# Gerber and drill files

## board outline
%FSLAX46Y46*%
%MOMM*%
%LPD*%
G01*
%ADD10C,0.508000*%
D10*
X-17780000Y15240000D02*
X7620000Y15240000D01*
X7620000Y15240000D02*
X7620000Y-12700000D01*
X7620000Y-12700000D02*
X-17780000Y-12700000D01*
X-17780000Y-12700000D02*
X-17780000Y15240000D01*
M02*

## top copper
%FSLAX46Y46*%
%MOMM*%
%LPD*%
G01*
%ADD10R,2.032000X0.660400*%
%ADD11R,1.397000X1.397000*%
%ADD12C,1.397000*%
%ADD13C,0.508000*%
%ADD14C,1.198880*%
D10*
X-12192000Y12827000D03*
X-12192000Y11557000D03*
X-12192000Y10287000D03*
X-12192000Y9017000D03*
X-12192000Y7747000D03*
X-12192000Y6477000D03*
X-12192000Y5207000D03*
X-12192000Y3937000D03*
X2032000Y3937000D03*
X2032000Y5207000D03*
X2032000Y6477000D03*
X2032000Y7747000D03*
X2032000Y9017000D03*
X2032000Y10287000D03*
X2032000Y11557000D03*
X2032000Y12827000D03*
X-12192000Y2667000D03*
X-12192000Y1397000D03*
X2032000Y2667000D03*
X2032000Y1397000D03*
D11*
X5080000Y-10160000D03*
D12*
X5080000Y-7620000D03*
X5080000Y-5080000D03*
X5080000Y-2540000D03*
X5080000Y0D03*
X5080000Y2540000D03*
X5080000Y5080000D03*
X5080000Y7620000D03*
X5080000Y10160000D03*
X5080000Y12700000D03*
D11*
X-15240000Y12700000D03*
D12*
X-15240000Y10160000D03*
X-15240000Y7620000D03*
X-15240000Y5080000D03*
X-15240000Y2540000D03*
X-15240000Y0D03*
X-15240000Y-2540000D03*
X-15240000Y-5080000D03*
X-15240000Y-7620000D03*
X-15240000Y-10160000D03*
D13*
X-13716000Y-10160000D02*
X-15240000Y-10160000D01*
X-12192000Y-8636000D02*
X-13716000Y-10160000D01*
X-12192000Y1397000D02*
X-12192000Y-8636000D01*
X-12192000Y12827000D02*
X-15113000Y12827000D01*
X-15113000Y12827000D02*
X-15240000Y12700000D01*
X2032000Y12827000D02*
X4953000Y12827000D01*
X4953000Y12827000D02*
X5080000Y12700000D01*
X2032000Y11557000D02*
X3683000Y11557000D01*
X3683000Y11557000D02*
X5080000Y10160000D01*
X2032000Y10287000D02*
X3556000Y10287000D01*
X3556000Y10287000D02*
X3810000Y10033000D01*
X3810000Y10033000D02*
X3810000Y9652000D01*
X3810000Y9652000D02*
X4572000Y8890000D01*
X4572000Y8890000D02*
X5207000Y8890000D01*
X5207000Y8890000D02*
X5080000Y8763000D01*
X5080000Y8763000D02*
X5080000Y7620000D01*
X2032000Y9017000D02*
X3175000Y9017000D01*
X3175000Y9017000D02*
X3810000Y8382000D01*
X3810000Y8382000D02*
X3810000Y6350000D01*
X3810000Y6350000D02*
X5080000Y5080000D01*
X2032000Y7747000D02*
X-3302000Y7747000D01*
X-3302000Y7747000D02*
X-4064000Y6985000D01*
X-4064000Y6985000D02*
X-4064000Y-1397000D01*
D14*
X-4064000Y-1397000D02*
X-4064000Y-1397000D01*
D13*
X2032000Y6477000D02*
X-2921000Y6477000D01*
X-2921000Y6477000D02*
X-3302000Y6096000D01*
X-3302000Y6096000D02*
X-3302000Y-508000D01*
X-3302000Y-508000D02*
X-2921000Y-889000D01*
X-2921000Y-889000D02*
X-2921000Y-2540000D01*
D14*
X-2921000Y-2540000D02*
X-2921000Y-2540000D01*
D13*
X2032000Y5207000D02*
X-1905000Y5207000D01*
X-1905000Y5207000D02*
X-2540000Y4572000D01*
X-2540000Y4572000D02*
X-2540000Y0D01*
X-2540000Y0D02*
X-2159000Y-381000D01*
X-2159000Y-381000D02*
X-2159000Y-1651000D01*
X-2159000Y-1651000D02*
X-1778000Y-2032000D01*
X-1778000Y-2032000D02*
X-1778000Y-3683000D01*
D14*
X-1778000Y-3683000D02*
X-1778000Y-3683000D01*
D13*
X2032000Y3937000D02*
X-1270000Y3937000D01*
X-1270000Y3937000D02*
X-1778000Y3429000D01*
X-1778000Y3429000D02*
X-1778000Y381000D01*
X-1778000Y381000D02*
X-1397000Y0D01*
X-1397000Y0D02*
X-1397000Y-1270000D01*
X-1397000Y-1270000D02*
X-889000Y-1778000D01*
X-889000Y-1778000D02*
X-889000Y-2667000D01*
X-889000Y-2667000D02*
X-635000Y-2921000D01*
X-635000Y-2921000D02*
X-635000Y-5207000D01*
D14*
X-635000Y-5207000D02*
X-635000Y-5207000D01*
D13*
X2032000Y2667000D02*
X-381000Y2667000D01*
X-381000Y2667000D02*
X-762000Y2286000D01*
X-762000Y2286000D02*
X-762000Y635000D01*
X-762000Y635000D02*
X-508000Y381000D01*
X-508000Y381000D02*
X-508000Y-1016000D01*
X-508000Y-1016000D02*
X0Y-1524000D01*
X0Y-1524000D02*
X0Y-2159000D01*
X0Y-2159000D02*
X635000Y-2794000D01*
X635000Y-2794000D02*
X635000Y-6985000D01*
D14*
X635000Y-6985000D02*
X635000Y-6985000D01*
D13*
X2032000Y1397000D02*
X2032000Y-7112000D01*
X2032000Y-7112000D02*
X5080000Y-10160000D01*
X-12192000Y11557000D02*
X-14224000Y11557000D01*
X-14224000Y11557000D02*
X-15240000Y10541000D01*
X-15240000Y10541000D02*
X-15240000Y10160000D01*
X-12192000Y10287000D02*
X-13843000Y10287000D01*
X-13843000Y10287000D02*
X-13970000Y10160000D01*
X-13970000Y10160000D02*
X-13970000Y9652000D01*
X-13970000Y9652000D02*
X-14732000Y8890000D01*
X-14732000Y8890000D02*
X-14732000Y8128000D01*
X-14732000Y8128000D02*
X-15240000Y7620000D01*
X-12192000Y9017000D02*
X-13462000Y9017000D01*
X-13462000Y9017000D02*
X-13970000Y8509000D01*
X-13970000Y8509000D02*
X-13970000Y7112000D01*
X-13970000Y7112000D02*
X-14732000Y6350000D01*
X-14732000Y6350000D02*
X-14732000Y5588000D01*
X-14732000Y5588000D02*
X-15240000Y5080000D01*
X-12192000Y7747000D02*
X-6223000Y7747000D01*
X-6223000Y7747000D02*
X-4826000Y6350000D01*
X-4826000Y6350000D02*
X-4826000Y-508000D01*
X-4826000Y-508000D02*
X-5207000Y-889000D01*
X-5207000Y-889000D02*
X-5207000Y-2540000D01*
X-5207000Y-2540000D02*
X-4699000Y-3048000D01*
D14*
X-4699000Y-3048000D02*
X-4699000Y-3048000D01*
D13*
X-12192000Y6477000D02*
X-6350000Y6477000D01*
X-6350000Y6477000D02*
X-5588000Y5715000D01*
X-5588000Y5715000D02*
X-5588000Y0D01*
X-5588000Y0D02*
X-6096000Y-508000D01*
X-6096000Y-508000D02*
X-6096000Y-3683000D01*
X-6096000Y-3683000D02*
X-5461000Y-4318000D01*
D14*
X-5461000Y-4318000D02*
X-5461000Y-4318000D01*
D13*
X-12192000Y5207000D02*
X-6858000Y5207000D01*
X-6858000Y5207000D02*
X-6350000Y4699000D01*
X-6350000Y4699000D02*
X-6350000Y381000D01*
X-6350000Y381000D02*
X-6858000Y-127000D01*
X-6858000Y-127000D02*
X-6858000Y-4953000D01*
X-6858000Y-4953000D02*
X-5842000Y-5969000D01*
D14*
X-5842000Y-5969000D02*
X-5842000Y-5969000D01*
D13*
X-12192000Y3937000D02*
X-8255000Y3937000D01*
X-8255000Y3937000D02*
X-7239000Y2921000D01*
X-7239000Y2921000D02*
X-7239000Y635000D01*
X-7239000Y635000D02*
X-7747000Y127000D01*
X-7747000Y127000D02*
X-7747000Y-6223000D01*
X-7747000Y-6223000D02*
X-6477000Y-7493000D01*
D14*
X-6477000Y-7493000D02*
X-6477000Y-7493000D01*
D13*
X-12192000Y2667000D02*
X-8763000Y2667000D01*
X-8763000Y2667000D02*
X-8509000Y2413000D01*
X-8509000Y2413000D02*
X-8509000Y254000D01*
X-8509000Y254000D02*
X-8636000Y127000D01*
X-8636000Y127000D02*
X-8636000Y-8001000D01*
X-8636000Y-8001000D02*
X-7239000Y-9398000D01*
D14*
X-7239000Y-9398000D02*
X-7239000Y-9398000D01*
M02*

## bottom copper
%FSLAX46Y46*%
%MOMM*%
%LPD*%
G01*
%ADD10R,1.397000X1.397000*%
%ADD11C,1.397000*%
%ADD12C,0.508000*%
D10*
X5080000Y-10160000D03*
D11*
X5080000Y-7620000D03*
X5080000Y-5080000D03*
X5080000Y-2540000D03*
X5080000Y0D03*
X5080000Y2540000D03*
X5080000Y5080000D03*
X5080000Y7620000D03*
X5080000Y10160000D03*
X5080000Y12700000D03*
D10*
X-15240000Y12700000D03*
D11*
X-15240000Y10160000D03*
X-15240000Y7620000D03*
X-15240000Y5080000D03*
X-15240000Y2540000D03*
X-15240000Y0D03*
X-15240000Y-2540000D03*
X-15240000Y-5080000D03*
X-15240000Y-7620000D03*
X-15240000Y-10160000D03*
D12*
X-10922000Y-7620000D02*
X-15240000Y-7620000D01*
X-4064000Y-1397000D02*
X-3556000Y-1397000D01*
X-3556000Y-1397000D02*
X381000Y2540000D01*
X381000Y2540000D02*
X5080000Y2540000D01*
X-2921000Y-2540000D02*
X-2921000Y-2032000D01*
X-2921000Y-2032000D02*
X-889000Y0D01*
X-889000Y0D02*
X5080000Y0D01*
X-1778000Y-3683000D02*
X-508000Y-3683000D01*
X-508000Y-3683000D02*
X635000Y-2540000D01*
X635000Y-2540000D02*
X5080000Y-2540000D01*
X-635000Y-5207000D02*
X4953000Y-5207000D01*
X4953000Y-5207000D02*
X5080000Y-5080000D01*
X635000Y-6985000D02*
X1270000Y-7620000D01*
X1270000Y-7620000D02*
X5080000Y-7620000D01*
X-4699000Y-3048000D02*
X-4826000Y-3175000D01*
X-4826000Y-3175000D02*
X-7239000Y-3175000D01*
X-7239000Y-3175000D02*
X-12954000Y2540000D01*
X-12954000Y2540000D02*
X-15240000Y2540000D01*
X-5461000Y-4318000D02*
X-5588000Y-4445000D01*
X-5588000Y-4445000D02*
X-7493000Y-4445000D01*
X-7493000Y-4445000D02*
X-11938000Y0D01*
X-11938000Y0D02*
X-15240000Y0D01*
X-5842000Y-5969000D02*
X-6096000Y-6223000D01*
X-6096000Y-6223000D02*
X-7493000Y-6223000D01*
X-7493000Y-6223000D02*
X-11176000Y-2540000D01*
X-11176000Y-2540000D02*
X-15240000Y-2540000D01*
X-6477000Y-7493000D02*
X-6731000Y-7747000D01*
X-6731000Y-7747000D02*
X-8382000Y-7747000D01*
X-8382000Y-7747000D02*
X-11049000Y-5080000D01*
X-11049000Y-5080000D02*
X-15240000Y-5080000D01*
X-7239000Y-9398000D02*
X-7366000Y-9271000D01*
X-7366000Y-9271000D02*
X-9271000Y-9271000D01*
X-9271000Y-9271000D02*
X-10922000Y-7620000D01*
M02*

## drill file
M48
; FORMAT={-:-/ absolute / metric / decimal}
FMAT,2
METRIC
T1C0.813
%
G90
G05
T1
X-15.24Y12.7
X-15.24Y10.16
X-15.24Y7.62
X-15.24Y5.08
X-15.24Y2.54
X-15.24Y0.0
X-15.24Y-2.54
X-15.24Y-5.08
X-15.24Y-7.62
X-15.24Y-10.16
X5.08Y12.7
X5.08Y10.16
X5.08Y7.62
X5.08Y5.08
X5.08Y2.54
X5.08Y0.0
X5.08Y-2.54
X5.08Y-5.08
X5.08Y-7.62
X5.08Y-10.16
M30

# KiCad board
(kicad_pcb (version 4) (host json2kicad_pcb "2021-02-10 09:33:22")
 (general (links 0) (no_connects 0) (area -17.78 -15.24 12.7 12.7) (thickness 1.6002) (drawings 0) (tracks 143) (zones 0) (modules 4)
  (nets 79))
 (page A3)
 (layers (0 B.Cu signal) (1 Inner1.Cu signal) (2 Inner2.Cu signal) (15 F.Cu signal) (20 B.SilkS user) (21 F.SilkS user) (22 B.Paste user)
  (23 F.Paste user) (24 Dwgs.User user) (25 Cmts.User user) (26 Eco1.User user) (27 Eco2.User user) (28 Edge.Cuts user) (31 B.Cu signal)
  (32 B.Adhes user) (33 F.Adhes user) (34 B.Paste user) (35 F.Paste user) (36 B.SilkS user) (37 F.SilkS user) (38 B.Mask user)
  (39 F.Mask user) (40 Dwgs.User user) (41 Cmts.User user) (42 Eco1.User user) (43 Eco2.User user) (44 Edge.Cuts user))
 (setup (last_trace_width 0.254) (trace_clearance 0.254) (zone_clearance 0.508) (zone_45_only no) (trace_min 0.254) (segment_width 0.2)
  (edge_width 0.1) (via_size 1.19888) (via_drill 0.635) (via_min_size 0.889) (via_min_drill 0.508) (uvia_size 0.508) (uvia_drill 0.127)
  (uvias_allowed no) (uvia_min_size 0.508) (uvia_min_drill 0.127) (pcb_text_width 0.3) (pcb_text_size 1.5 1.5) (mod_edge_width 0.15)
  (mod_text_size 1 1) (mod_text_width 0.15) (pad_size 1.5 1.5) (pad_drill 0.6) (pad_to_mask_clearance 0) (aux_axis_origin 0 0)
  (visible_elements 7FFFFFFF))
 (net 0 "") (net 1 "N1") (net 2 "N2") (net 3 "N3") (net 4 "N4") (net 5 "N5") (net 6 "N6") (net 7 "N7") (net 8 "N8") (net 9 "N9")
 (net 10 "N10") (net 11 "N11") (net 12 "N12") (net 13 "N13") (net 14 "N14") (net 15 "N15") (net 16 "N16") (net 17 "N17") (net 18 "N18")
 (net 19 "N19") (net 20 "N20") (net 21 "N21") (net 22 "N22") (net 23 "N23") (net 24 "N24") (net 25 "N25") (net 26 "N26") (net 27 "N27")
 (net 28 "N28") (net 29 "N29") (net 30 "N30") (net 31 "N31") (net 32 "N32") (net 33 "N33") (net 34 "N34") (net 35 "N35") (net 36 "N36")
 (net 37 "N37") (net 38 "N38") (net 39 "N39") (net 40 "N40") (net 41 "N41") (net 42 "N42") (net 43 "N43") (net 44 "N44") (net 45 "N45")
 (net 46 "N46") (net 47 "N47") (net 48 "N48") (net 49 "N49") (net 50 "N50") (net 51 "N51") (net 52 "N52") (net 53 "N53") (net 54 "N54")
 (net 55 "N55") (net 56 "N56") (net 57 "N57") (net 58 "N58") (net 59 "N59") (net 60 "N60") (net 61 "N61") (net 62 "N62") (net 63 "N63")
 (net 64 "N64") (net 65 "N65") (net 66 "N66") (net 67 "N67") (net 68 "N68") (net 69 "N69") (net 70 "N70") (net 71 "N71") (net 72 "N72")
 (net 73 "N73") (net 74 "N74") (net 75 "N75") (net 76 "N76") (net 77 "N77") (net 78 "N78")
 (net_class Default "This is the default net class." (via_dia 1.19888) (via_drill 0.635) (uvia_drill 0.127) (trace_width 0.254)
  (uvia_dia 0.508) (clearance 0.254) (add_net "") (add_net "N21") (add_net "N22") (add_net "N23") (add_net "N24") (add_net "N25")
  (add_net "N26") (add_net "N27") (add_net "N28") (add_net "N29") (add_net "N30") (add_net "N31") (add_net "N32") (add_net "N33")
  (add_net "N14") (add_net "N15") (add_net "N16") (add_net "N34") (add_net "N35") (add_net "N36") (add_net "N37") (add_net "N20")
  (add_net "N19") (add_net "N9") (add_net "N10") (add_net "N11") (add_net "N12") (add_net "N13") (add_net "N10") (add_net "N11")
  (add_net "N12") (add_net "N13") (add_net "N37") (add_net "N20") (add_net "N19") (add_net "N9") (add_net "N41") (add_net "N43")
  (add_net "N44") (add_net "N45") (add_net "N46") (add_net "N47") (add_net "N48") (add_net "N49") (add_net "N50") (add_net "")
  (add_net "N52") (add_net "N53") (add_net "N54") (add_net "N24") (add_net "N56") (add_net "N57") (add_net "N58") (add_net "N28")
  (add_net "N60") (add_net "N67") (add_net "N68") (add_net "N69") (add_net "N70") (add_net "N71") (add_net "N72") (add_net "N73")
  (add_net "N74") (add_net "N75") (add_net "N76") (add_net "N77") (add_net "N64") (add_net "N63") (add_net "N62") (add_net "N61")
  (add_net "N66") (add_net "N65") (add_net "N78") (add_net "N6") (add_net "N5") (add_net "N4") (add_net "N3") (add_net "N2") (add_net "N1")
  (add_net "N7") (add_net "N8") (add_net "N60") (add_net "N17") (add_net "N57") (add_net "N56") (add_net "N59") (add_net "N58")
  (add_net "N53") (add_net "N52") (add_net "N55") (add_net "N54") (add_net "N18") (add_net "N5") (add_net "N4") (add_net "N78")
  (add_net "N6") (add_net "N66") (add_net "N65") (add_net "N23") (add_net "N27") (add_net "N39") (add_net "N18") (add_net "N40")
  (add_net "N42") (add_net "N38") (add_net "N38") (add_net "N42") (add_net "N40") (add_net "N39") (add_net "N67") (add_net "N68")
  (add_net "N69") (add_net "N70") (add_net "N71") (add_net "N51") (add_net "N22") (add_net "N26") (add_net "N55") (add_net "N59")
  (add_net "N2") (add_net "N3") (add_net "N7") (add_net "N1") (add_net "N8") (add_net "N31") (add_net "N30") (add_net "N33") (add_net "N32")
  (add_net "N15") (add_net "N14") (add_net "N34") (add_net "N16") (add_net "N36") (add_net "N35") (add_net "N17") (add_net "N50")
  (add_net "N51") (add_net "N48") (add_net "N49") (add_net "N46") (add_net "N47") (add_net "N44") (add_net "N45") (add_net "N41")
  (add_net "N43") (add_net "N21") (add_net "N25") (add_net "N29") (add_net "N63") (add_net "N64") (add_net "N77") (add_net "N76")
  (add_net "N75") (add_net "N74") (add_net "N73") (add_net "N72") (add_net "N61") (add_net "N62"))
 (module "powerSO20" (layer "F.Cu") (at -5.08 -7.112 -90.00)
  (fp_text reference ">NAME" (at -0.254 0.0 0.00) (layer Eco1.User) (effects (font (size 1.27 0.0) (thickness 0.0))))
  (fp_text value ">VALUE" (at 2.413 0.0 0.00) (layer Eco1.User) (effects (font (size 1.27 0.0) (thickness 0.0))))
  (pad 1 smd rect (at -5.715 7.112 -90.00) (size 0.6604 2.032) (drill 0.0) (layers "F.Cu" "F.Paste") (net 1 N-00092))
  (pad 2 smd rect (at -4.445 7.112 -90.00) (size 0.6604 2.032) (drill 0.0) (layers "F.Cu" "F.Paste") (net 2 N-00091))
  (pad 3 smd rect (at -3.175 7.112 -90.00) (size 0.6604 2.032) (drill 0.0) (layers "F.Cu" "F.Paste") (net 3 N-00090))
  (pad 4 smd rect (at -1.905 7.112 -90.00) (size 0.6604 2.032) (drill 0.0) (layers "F.Cu" "F.Paste") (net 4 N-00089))
  (pad 5 smd rect (at -0.635 7.112 -90.00) (size 0.6604 2.032) (drill 0.0) (layers "F.Cu" "F.Paste") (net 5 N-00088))
  (pad 6 smd rect (at 0.635 7.112 -90.00) (size 0.6604 2.032) (drill 0.0) (layers "F.Cu" "F.Paste") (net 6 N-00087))
  (pad 7 smd rect (at 1.905 7.112 -90.00) (size 0.6604 2.032) (drill 0.0) (layers "F.Cu" "F.Paste") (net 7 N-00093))
  (pad 8 smd rect (at 3.175 7.112 -90.00) (size 0.6604 2.032) (drill 0.0) (layers "F.Cu" "F.Paste") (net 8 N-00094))
  (pad 13 smd rect (at 3.175 -7.112 -90.00) (size 0.6604 2.032) (drill 0.0) (layers "F.Cu" "F.Paste") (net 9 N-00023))
  (pad 14 smd rect (at 1.905 -7.112 -90.00) (size 0.6604 2.032) (drill 0.0) (layers "F.Cu" "F.Paste") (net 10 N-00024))
  (pad 15 smd rect (at 0.635 -7.112 -90.00) (size 0.6604 2.032) (drill 0.0) (layers "F.Cu" "F.Paste") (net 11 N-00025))
  (pad 16 smd rect (at -0.635 -7.112 -90.00) (size 0.6604 2.032) (drill 0.0) (layers "F.Cu" "F.Paste") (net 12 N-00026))
  (pad 17 smd rect (at -1.905 -7.112 -90.00) (size 0.6604 2.032) (drill 0.0) (layers "F.Cu" "F.Paste") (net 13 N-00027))
  (pad 18 smd rect (at -3.175 -7.112 -90.00) (size 0.6604 2.032) (drill 0.0) (layers "F.Cu" "F.Paste") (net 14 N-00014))
  (pad 19 smd rect (at -4.445 -7.112 -90.00) (size 0.6604 2.032) (drill 0.0) (layers "F.Cu" "F.Paste") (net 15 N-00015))
  (pad 20 smd rect (at -5.715 -7.112 -90.00) (size 0.6604 2.032) (drill 0.0) (layers "F.Cu" "F.Paste") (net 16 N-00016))
  (pad 9 smd rect (at 4.445 7.112 -90.00) (size 0.6604 2.032) (drill 0.0) (layers "F.Cu" "F.Paste") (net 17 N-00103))
  (pad 10 smd rect (at 5.715 7.112 -90.00) (size 0.6604 2.032) (drill 0.0) (layers "F.Cu" "F.Paste") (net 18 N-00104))
  (pad 12 smd rect (at 4.445 -7.112 -90.00) (size 0.6604 2.032) (drill 0.0) (layers "F.Cu" "F.Paste") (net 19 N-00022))
  (pad 11 smd rect (at 5.715 -7.112 -90.00) (size 0.6604 2.032) (drill 0.0) (layers "F.Cu" "F.Paste") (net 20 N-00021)))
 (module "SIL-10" (layer "F.Cu") (at 5.08 -1.27 90.00)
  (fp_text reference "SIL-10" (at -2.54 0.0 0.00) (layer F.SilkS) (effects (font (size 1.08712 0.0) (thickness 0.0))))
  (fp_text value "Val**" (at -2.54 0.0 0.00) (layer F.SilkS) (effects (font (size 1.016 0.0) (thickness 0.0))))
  (pad 1 thru_hole rect (at -11.43 0.0 90.00) (size 1.397 1.397) (drill 0.8128)
   (layers "B.Cu" "Inner1.Cu" "Inner2.Cu" "F.Cu" "F.SilkS" "B.Paste" "F.Paste") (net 20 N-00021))
  (pad 2 thru_hole circle (at -8.89 0.0 90.00) (size 1.397 1.397) (drill 0.8128)
   (layers "B.Cu" "Inner1.Cu" "Inner2.Cu" "F.Cu" "F.SilkS" "B.Paste" "F.Paste") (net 19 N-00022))
  (pad 3 thru_hole circle (at -6.35 0.0 90.00) (size 1.397 1.397) (drill 0.8128)
   (layers "B.Cu" "Inner1.Cu" "Inner2.Cu" "F.Cu" "F.SilkS" "B.Paste" "F.Paste") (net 9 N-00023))
  (pad 4 thru_hole circle (at -3.81 0.0 90.00) (size 1.397 1.397) (drill 0.8128)
   (layers "B.Cu" "Inner1.Cu" "Inner2.Cu" "F.Cu" "F.SilkS" "B.Paste" "F.Paste") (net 10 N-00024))
  (pad 5 thru_hole circle (at -1.27 0.0 90.00) (size 1.397 1.397) (drill 0.8128)
   (layers "B.Cu" "Inner1.Cu" "Inner2.Cu" "F.Cu" "F.SilkS" "B.Paste" "F.Paste") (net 11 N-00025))
  (pad 6 thru_hole circle (at 1.27 0.0 90.00) (size 1.397 1.397) (drill 0.8128)
   (layers "B.Cu" "Inner1.Cu" "Inner2.Cu" "F.Cu" "F.SilkS" "B.Paste" "F.Paste") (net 12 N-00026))
  (pad 7 thru_hole circle (at 3.81 0.0 90.00) (size 1.397 1.397) (drill 0.8128)
   (layers "B.Cu" "Inner1.Cu" "Inner2.Cu" "F.Cu" "F.SilkS" "B.Paste" "F.Paste") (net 13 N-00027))
  (pad 8 thru_hole circle (at 6.35 0.0 90.00) (size 1.397 1.397) (drill 0.8128)
   (layers "B.Cu" "Inner1.Cu" "Inner2.Cu" "F.Cu" "F.SilkS" "B.Paste" "F.Paste") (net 14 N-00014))
  (pad 9 thru_hole circle (at 8.89 0.0 90.00) (size 1.397 1.397) (drill 0.8128)
   (layers "B.Cu" "Inner1.Cu" "Inner2.Cu" "F.Cu" "F.SilkS" "B.Paste" "F.Paste") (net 15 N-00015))
  (pad 10 thru_hole circle (at 11.43 0.0 90.00) (size 1.397 1.397) (drill 0.8128)
   (layers "B.Cu" "Inner1.Cu" "Inner2.Cu" "F.Cu" "F.SilkS" "B.Paste" "F.Paste") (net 16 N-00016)))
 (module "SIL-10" (layer "F.Cu") (at -15.24 -1.27 -90.00)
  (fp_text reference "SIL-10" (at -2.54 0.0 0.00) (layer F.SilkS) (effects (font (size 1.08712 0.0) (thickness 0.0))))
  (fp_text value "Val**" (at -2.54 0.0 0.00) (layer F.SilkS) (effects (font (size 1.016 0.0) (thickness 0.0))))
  (pad 1 thru_hole rect (at -11.43 0.0 -90.00) (size 1.397 1.397) (drill 0.8128)
   (layers "B.Cu" "Inner1.Cu" "Inner2.Cu" "F.Cu" "F.SilkS" "B.Paste" "F.Paste") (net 1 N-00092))
  (pad 2 thru_hole circle (at -8.89 0.0 -90.00) (size 1.397 1.397) (drill 0.8128)
   (layers "B.Cu" "Inner1.Cu" "Inner2.Cu" "F.Cu" "F.SilkS" "B.Paste" "F.Paste") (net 2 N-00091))
  (pad 3 thru_hole circle (at -6.35 0.0 -90.00) (size 1.397 1.397) (drill 0.8128)
   (layers "B.Cu" "Inner1.Cu" "Inner2.Cu" "F.Cu" "F.SilkS" "B.Paste" "F.Paste") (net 3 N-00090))
  (pad 4 thru_hole circle (at -3.81 0.0 -90.00) (size 1.397 1.397) (drill 0.8128)
   (layers "B.Cu" "Inner1.Cu" "Inner2.Cu" "F.Cu" "F.SilkS" "B.Paste" "F.Paste") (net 4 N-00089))
  (pad 5 thru_hole circle (at -1.27 0.0 -90.00) (size 1.397 1.397) (drill 0.8128)
   (layers "B.Cu" "Inner1.Cu" "Inner2.Cu" "F.Cu" "F.SilkS" "B.Paste" "F.Paste") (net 5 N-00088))
  (pad 6 thru_hole circle (at 1.27 0.0 -90.00) (size 1.397 1.397) (drill 0.8128)
   (layers "B.Cu" "Inner1.Cu" "Inner2.Cu" "F.Cu" "F.SilkS" "B.Paste" "F.Paste") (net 6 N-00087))
  (pad 7 thru_hole circle (at 3.81 0.0 -90.00) (size 1.397 1.397) (drill 0.8128)
   (layers "B.Cu" "Inner1.Cu" "Inner2.Cu" "F.Cu" "F.SilkS" "B.Paste" "F.Paste") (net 7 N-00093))
  (pad 8 thru_hole circle (at 6.35 0.0 -90.00) (size 1.397 1.397) (drill 0.8128)
   (layers "B.Cu" "Inner1.Cu" "Inner2.Cu" "F.Cu" "F.SilkS" "B.Paste" "F.Paste") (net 8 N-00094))
  (pad 9 thru_hole circle (at 8.89 0.0 -90.00) (size 1.397 1.397) (drill 0.8128)
   (layers "B.Cu" "Inner1.Cu" "Inner2.Cu" "F.Cu" "F.SilkS" "B.Paste" "F.Paste") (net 17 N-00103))
  (pad 10 thru_hole circle (at 11.43 0.0 -90.00) (size 1.397 1.397) (drill 0.8128)
   (layers "B.Cu" "Inner1.Cu" "Inner2.Cu" "F.Cu" "F.SilkS" "B.Paste" "F.Paste") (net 18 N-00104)))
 (segment (start -13.716 10.16) (end -15.24 10.16) (width 0.508) (layer F.Cu) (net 18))
 (segment (start -12.192 8.636) (end -13.716 10.16) (width 0.508) (layer F.Cu) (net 18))
 (segment (start -12.192 -1.397) (end -12.192 8.636) (width 0.508) (layer F.Cu) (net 18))
 (segment (start -10.922 7.62) (end -15.24 7.62) (width 0.508) (layer B.Cu) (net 17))
 (segment (start -12.192 -12.827) (end -15.113 -12.827) (width 0.508) (layer F.Cu) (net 1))
 (segment (start -15.113 -12.827) (end -15.24 -12.7) (width 0.508) (layer F.Cu) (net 1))
 (segment (start 2.032 -12.827) (end 4.953 -12.827) (width 0.508) (layer F.Cu) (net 16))
 (segment (start 4.953 -12.827) (end 5.08 -12.7) (width 0.508) (layer F.Cu) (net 16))
 (segment (start 2.032 -11.557) (end 3.683 -11.557) (width 0.508) (layer F.Cu) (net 15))
 (segment (start 3.683 -11.557) (end 5.08 -10.16) (width 0.508) (layer F.Cu) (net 15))
 (segment (start 2.032 -10.287) (end 3.556 -10.287) (width 0.508) (layer F.Cu) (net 14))
 (segment (start 3.556 -10.287) (end 3.81 -10.033) (width 0.508) (layer F.Cu) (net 14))
 (segment (start 3.81 -10.033) (end 3.81 -9.652) (width 0.508) (layer F.Cu) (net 14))
 (segment (start 3.81 -9.652) (end 4.572 -8.89) (width 0.508) (layer F.Cu) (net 14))
 (segment (start 4.572 -8.89) (end 5.207 -8.89) (width 0.508) (layer F.Cu) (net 14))
 (segment (start 5.207 -8.89) (end 5.08 -8.763) (width 0.508) (layer F.Cu) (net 14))
 (segment (start 5.08 -8.763) (end 5.08 -7.62) (width 0.508) (layer F.Cu) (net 14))
 (segment (start 2.032 -9.017) (end 3.175 -9.017) (width 0.508) (layer F.Cu) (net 13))
 (segment (start 3.175 -9.017) (end 3.81 -8.382) (width 0.508) (layer F.Cu) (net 13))
 (segment (start 3.81 -8.382) (end 3.81 -6.35) (width 0.508) (layer F.Cu) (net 13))
 (segment (start 3.81 -6.35) (end 5.08 -5.08) (width 0.508) (layer F.Cu) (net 13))
 (segment (start 2.032 -7.747) (end -3.302 -7.747) (width 0.508) (layer F.Cu) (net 12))
 (segment (start -3.302 -7.747) (end -4.064 -6.985) (width 0.508) (layer F.Cu) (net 12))
 (segment (start -4.064 -6.985) (end -4.064 1.397) (width 0.508) (layer F.Cu) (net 12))
 (segment (start -4.064 1.397) (end -4.064 1.397) (width 1.19888) (layer F.Cu) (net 12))
 (segment (start -4.064 1.397) (end -3.556 1.397) (width 0.508) (layer B.Cu) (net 12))
 (segment (start -3.556 1.397) (end 0.381 -2.54) (width 0.508) (layer B.Cu) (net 12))
 (segment (start 0.381 -2.54) (end 5.08 -2.54) (width 0.508) (layer B.Cu) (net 12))
 (segment (start 2.032 -6.477) (end -2.921 -6.477) (width 0.508) (layer F.Cu) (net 11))
 (segment (start -2.921 -6.477) (end -3.302 -6.096) (width 0.508) (layer F.Cu) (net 11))
 (segment (start -3.302 -6.096) (end -3.302 0.508) (width 0.508) (layer F.Cu) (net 11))
 (segment (start -3.302 0.508) (end -2.921 0.889) (width 0.508) (layer F.Cu) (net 11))
 (segment (start -2.921 0.889) (end -2.921 2.54) (width 0.508) (layer F.Cu) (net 11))
 (segment (start -2.921 2.54) (end -2.921 2.54) (width 1.19888) (layer F.Cu) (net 11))
 (segment (start -2.921 2.54) (end -2.921 2.032) (width 0.508) (layer B.Cu) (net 11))
 (segment (start -2.921 2.032) (end -0.889 0.0) (width 0.508) (layer B.Cu) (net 11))
 (segment (start -0.889 0.0) (end 5.08 0.0) (width 0.508) (layer B.Cu) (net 11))
 (segment (start 2.032 -5.207) (end -1.905 -5.207) (width 0.508) (layer F.Cu) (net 10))
 (segment (start -1.905 -5.207) (end -2.54 -4.572) (width 0.508) (layer F.Cu) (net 10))
 (segment (start -2.54 -4.572) (end -2.54 0.0) (width 0.508) (layer F.Cu) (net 10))
 (segment (start -2.54 0.0) (end -2.159 0.381) (width 0.508) (layer F.Cu) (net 10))
 (segment (start -2.159 0.381) (end -2.159 1.651) (width 0.508) (layer F.Cu) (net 10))
 (segment (start -2.159 1.651) (end -1.778 2.032) (width 0.508) (layer F.Cu) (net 10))
 (segment (start -1.778 2.032) (end -1.778 3.683) (width 0.508) (layer F.Cu) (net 10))
 (segment (start -1.778 3.683) (end -1.778 3.683) (width 1.19888) (layer F.Cu) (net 10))
 (segment (start -1.778 3.683) (end -0.508 3.683) (width 0.508) (layer B.Cu) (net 10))
 (segment (start -0.508 3.683) (end 0.635 2.54) (width 0.508) (layer B.Cu) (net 10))
 (segment (start 0.635 2.54) (end 5.08 2.54) (width 0.508) (layer B.Cu) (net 10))
 (segment (start 2.032 -3.937) (end -1.27 -3.937) (width 0.508) (layer F.Cu) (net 9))
 (segment (start -1.27 -3.937) (end -1.778 -3.429) (width 0.508) (layer F.Cu) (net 9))
 (segment (start -1.778 -3.429) (end -1.778 -0.381) (width 0.508) (layer F.Cu) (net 9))
 (segment (start -1.778 -0.381) (end -1.397 0.0) (width 0.508) (layer F.Cu) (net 9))
 (segment (start -1.397 0.0) (end -1.397 1.27) (width 0.508) (layer F.Cu) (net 9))
 (segment (start -1.397 1.27) (end -0.889 1.778) (width 0.508) (layer F.Cu) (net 9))
 (segment (start -0.889 1.778) (end -0.889 2.667) (width 0.508) (layer F.Cu) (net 9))
 (segment (start -0.889 2.667) (end -0.635 2.921) (width 0.508) (layer F.Cu) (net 9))
 (segment (start -0.635 2.921) (end -0.635 5.207) (width 0.508) (layer F.Cu) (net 9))
 (segment (start -0.635 5.207) (end -0.635 5.207) (width 1.19888) (layer F.Cu) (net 9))
 (segment (start -0.635 5.207) (end 4.953 5.207) (width 0.508) (layer B.Cu) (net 9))
 (segment (start 4.953 5.207) (end 5.08 5.08) (width 0.508) (layer B.Cu) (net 9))
 (segment (start 2.032 -2.667) (end -0.381 -2.667) (width 0.508) (layer F.Cu) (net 19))
 (segment (start -0.381 -2.667) (end -0.762 -2.286) (width 0.508) (layer F.Cu) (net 19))
 (segment (start -0.762 -2.286) (end -0.762 -0.635) (width 0.508) (layer F.Cu) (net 19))
 (segment (start -0.762 -0.635) (end -0.508 -0.381) (width 0.508) (layer F.Cu) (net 19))
 (segment (start -0.508 -0.381) (end -0.508 1.016) (width 0.508) (layer F.Cu) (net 19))
 (segment (start -0.508 1.016) (end 0.0 1.524) (width 0.508) (layer F.Cu) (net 19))
 (segment (start 0.0 1.524) (end 0.0 2.159) (width 0.508) (layer F.Cu) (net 19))
 (segment (start 0.0 2.159) (end 0.635 2.794) (width 0.508) (layer F.Cu) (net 19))
 (segment (start 0.635 2.794) (end 0.635 6.985) (width 0.508) (layer F.Cu) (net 19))
 (segment (start 0.635 6.985) (end 0.635 6.985) (width 1.19888) (layer F.Cu) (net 19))
 (segment (start 0.635 6.985) (end 1.27 7.62) (width 0.508) (layer B.Cu) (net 19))
 (segment (start 1.27 7.62) (end 5.08 7.62) (width 0.508) (layer B.Cu) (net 19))
 (segment (start 2.032 -1.397) (end 2.032 7.112) (width 0.508) (layer F.Cu) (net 20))
 (segment (start 2.032 7.112) (end 5.08 10.16) (width 0.508) (layer F.Cu) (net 20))
 (segment (start -12.192 -11.557) (end -14.224 -11.557) (width 0.508) (layer F.Cu) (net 2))
 (segment (start -14.224 -11.557) (end -15.24 -10.541) (width 0.508) (layer F.Cu) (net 2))
 (segment (start -15.24 -10.541) (end -15.24 -10.16) (width 0.508) (layer F.Cu) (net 2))
 (segment (start -12.192 -10.287) (end -13.843 -10.287) (width 0.508) (layer F.Cu) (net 3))
 (segment (start -13.843 -10.287) (end -13.97 -10.16) (width 0.508) (layer F.Cu) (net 3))
 (segment (start -13.97 -10.16) (end -13.97 -9.652) (width 0.508) (layer F.Cu) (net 3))
 (segment (start -13.97 -9.652) (end -14.732 -8.89) (width 0.508) (layer F.Cu) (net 3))
 (segment (start -14.732 -8.89) (end -14.732 -8.128) (width 0.508) (layer F.Cu) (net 3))
 (segment (start -14.732 -8.128) (end -15.24 -7.62) (width 0.508) (layer F.Cu) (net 3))
 (segment (start -12.192 -9.017) (end -13.462 -9.017) (width 0.508) (layer F.Cu) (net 4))
 (segment (start -13.462 -9.017) (end -13.97 -8.509) (width 0.508) (layer F.Cu) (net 4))
 (segment (start -13.97 -8.509) (end -13.97 -7.112) (width 0.508) (layer F.Cu) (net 4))
 (segment (start -13.97 -7.112) (end -14.732 -6.35) (width 0.508) (layer F.Cu) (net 4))
 (segment (start -14.732 -6.35) (end -14.732 -5.588) (width 0.508) (layer F.Cu) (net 4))
 (segment (start -14.732 -5.588) (end -15.24 -5.08) (width 0.508) (layer F.Cu) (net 4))
 (segment (start -12.192 -7.747) (end -6.223 -7.747) (width 0.508) (layer F.Cu) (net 5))
 (segment (start -6.223 -7.747) (end -4.826 -6.35) (width 0.508) (layer F.Cu) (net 5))
 (segment (start -4.826 -6.35) (end -4.826 0.508) (width 0.508) (layer F.Cu) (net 5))
 (segment (start -4.826 0.508) (end -5.207 0.889) (width 0.508) (layer F.Cu) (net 5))
 (segment (start -5.207 0.889) (end -5.207 2.54) (width 0.508) (layer F.Cu) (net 5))
 (segment (start -5.207 2.54) (end -4.699 3.048) (width 0.508) (layer F.Cu) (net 5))
 (segment (start -4.699 3.048) (end -4.699 3.048) (width 1.19888) (layer F.Cu) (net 5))
 (segment (start -4.699 3.048) (end -4.826 3.175) (width 0.508) (layer B.Cu) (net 5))
 (segment (start -4.826 3.175) (end -7.239 3.175) (width 0.508) (layer B.Cu) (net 5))
 (segment (start -7.239 3.175) (end -12.954 -2.54) (width 0.508) (layer B.Cu) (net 5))
 (segment (start -12.954 -2.54) (end -15.24 -2.54) (width 0.508) (layer B.Cu) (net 5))
 (segment (start -12.192 -6.477) (end -6.35 -6.477) (width 0.508) (layer F.Cu) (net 6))
 (segment (start -6.35 -6.477) (end -5.588 -5.715) (width 0.508) (layer F.Cu) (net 6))
 (segment (start -5.588 -5.715) (end -5.588 0.0) (width 0.508) (layer F.Cu) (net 6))
 (segment (start -5.588 0.0) (end -6.096 0.508) (width 0.508) (layer F.Cu) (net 6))
 (segment (start -6.096 0.508) (end -6.096 3.683) (width 0.508) (layer F.Cu) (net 6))
 (segment (start -6.096 3.683) (end -5.461 4.318) (width 0.508) (layer F.Cu) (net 6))
 (segment (start -5.461 4.318) (end -5.461 4.318) (width 1.19888) (layer F.Cu) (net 6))
 (segment (start -5.461 4.318) (end -5.588 4.445) (width 0.508) (layer B.Cu) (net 6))
 (segment (start -5.588 4.445) (end -7.493 4.445) (width 0.508) (layer B.Cu) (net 6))
 (segment (start -7.493 4.445) (end -11.938 0.0) (width 0.508) (layer B.Cu) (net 6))
 (segment (start -11.938 0.0) (end -15.24 0.0) (width 0.508) (layer B.Cu) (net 6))
 (segment (start -12.192 -5.207) (end -6.858 -5.207) (width 0.508) (layer F.Cu) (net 7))
 (segment (start -6.858 -5.207) (end -6.35 -4.699) (width 0.508) (layer F.Cu) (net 7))
 (segment (start -6.35 -4.699) (end -6.35 -0.381) (width 0.508) (layer F.Cu) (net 7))
 (segment (start -6.35 -0.381) (end -6.858 0.127) (width 0.508) (layer F.Cu) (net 7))
 (segment (start -6.858 0.127) (end -6.858 4.953) (width 0.508) (layer F.Cu) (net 7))
 (segment (start -6.858 4.953) (end -5.842 5.969) (width 0.508) (layer F.Cu) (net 7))
 (segment (start -5.842 5.969) (end -5.842 5.969) (width 1.19888) (layer F.Cu) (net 7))
 (segment (start -5.842 5.969) (end -6.096 6.223) (width 0.508) (layer B.Cu) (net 7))
 (segment (start -6.096 6.223) (end -7.493 6.223) (width 0.508) (layer B.Cu) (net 7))
 (segment (start -7.493 6.223) (end -11.176 2.54) (width 0.508) (layer B.Cu) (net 7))
 (segment (start -11.176 2.54) (end -15.24 2.54) (width 0.508) (layer B.Cu) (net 7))
 (segment (start -12.192 -3.937) (end -8.255 -3.937) (width 0.508) (layer F.Cu) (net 8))
 (segment (start -8.255 -3.937) (end -7.239 -2.921) (width 0.508) (layer F.Cu) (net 8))
 (segment (start -7.239 -2.921) (end -7.239 -0.635) (width 0.508) (layer F.Cu) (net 8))
 (segment (start -7.239 -0.635) (end -7.747 -0.127) (width 0.508) (layer F.Cu) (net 8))
 (segment (start -7.747 -0.127) (end -7.747 6.223) (width 0.508) (layer F.Cu) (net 8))
 (segment (start -7.747 6.223) (end -6.477 7.493) (width 0.508) (layer F.Cu) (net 8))
 (segment (start -6.477 7.493) (end -6.477 7.493) (width 1.19888) (layer F.Cu) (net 8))
 (segment (start -6.477 7.493) (end -6.731 7.747) (width 0.508) (layer B.Cu) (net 8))
 (segment (start -6.731 7.747) (end -8.382 7.747) (width 0.508) (layer B.Cu) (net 8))
 (segment (start -8.382 7.747) (end -11.049 5.08) (width 0.508) (layer B.Cu) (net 8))
 (segment (start -11.049 5.08) (end -15.24 5.08) (width 0.508) (layer B.Cu) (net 8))
 (segment (start -12.192 -2.667) (end -8.763 -2.667) (width 0.508) (layer F.Cu) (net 17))
 (segment (start -8.763 -2.667) (end -8.509 -2.413) (width 0.508) (layer F.Cu) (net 17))
 (segment (start -8.509 -2.413) (end -8.509 -0.254) (width 0.508) (layer F.Cu) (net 17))
 (segment (start -8.509 -0.254) (end -8.636 -0.127) (width 0.508) (layer F.Cu) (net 17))
 (segment (start -8.636 -0.127) (end -8.636 8.001) (width 0.508) (layer F.Cu) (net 17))
 (segment (start -8.636 8.001) (end -7.239 9.398) (width 0.508) (layer F.Cu) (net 17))
 (segment (start -7.239 9.398) (end -7.239 9.398) (width 1.19888) (layer F.Cu) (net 17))
 (segment (start -7.239 9.398) (end -7.366 9.271) (width 0.508) (layer B.Cu) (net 17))
 (segment (start -7.366 9.271) (end -9.271 9.271) (width 0.508) (layer B.Cu) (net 17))
 (segment (start -9.271 9.271) (end -10.922 7.62) (width 0.508) (layer B.Cu) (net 17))
 (gr_line (start -17.78 -15.24) (end 7.62 -15.24) (angle 51566.20) (width 0.508) (layer Edge.Cuts))
 (gr_line (start 7.62 -15.24) (end 7.62 12.7) (angle 51566.20) (width 0.508) (layer Edge.Cuts))
 (gr_line (start 7.62 12.7) (end -17.78 12.7) (angle 51566.20) (width 0.508) (layer Edge.Cuts))
 (gr_line (start -17.78 12.7) (end -17.78 -15.24) (angle 51566.20) (width 0.508) (layer Edge.Cuts))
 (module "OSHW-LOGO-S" (layer "F.Cu") (at -2.413 9.398 0.00)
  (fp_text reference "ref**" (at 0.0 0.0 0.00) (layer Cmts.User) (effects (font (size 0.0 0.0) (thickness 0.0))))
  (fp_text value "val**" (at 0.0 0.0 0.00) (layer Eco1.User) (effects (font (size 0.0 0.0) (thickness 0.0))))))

